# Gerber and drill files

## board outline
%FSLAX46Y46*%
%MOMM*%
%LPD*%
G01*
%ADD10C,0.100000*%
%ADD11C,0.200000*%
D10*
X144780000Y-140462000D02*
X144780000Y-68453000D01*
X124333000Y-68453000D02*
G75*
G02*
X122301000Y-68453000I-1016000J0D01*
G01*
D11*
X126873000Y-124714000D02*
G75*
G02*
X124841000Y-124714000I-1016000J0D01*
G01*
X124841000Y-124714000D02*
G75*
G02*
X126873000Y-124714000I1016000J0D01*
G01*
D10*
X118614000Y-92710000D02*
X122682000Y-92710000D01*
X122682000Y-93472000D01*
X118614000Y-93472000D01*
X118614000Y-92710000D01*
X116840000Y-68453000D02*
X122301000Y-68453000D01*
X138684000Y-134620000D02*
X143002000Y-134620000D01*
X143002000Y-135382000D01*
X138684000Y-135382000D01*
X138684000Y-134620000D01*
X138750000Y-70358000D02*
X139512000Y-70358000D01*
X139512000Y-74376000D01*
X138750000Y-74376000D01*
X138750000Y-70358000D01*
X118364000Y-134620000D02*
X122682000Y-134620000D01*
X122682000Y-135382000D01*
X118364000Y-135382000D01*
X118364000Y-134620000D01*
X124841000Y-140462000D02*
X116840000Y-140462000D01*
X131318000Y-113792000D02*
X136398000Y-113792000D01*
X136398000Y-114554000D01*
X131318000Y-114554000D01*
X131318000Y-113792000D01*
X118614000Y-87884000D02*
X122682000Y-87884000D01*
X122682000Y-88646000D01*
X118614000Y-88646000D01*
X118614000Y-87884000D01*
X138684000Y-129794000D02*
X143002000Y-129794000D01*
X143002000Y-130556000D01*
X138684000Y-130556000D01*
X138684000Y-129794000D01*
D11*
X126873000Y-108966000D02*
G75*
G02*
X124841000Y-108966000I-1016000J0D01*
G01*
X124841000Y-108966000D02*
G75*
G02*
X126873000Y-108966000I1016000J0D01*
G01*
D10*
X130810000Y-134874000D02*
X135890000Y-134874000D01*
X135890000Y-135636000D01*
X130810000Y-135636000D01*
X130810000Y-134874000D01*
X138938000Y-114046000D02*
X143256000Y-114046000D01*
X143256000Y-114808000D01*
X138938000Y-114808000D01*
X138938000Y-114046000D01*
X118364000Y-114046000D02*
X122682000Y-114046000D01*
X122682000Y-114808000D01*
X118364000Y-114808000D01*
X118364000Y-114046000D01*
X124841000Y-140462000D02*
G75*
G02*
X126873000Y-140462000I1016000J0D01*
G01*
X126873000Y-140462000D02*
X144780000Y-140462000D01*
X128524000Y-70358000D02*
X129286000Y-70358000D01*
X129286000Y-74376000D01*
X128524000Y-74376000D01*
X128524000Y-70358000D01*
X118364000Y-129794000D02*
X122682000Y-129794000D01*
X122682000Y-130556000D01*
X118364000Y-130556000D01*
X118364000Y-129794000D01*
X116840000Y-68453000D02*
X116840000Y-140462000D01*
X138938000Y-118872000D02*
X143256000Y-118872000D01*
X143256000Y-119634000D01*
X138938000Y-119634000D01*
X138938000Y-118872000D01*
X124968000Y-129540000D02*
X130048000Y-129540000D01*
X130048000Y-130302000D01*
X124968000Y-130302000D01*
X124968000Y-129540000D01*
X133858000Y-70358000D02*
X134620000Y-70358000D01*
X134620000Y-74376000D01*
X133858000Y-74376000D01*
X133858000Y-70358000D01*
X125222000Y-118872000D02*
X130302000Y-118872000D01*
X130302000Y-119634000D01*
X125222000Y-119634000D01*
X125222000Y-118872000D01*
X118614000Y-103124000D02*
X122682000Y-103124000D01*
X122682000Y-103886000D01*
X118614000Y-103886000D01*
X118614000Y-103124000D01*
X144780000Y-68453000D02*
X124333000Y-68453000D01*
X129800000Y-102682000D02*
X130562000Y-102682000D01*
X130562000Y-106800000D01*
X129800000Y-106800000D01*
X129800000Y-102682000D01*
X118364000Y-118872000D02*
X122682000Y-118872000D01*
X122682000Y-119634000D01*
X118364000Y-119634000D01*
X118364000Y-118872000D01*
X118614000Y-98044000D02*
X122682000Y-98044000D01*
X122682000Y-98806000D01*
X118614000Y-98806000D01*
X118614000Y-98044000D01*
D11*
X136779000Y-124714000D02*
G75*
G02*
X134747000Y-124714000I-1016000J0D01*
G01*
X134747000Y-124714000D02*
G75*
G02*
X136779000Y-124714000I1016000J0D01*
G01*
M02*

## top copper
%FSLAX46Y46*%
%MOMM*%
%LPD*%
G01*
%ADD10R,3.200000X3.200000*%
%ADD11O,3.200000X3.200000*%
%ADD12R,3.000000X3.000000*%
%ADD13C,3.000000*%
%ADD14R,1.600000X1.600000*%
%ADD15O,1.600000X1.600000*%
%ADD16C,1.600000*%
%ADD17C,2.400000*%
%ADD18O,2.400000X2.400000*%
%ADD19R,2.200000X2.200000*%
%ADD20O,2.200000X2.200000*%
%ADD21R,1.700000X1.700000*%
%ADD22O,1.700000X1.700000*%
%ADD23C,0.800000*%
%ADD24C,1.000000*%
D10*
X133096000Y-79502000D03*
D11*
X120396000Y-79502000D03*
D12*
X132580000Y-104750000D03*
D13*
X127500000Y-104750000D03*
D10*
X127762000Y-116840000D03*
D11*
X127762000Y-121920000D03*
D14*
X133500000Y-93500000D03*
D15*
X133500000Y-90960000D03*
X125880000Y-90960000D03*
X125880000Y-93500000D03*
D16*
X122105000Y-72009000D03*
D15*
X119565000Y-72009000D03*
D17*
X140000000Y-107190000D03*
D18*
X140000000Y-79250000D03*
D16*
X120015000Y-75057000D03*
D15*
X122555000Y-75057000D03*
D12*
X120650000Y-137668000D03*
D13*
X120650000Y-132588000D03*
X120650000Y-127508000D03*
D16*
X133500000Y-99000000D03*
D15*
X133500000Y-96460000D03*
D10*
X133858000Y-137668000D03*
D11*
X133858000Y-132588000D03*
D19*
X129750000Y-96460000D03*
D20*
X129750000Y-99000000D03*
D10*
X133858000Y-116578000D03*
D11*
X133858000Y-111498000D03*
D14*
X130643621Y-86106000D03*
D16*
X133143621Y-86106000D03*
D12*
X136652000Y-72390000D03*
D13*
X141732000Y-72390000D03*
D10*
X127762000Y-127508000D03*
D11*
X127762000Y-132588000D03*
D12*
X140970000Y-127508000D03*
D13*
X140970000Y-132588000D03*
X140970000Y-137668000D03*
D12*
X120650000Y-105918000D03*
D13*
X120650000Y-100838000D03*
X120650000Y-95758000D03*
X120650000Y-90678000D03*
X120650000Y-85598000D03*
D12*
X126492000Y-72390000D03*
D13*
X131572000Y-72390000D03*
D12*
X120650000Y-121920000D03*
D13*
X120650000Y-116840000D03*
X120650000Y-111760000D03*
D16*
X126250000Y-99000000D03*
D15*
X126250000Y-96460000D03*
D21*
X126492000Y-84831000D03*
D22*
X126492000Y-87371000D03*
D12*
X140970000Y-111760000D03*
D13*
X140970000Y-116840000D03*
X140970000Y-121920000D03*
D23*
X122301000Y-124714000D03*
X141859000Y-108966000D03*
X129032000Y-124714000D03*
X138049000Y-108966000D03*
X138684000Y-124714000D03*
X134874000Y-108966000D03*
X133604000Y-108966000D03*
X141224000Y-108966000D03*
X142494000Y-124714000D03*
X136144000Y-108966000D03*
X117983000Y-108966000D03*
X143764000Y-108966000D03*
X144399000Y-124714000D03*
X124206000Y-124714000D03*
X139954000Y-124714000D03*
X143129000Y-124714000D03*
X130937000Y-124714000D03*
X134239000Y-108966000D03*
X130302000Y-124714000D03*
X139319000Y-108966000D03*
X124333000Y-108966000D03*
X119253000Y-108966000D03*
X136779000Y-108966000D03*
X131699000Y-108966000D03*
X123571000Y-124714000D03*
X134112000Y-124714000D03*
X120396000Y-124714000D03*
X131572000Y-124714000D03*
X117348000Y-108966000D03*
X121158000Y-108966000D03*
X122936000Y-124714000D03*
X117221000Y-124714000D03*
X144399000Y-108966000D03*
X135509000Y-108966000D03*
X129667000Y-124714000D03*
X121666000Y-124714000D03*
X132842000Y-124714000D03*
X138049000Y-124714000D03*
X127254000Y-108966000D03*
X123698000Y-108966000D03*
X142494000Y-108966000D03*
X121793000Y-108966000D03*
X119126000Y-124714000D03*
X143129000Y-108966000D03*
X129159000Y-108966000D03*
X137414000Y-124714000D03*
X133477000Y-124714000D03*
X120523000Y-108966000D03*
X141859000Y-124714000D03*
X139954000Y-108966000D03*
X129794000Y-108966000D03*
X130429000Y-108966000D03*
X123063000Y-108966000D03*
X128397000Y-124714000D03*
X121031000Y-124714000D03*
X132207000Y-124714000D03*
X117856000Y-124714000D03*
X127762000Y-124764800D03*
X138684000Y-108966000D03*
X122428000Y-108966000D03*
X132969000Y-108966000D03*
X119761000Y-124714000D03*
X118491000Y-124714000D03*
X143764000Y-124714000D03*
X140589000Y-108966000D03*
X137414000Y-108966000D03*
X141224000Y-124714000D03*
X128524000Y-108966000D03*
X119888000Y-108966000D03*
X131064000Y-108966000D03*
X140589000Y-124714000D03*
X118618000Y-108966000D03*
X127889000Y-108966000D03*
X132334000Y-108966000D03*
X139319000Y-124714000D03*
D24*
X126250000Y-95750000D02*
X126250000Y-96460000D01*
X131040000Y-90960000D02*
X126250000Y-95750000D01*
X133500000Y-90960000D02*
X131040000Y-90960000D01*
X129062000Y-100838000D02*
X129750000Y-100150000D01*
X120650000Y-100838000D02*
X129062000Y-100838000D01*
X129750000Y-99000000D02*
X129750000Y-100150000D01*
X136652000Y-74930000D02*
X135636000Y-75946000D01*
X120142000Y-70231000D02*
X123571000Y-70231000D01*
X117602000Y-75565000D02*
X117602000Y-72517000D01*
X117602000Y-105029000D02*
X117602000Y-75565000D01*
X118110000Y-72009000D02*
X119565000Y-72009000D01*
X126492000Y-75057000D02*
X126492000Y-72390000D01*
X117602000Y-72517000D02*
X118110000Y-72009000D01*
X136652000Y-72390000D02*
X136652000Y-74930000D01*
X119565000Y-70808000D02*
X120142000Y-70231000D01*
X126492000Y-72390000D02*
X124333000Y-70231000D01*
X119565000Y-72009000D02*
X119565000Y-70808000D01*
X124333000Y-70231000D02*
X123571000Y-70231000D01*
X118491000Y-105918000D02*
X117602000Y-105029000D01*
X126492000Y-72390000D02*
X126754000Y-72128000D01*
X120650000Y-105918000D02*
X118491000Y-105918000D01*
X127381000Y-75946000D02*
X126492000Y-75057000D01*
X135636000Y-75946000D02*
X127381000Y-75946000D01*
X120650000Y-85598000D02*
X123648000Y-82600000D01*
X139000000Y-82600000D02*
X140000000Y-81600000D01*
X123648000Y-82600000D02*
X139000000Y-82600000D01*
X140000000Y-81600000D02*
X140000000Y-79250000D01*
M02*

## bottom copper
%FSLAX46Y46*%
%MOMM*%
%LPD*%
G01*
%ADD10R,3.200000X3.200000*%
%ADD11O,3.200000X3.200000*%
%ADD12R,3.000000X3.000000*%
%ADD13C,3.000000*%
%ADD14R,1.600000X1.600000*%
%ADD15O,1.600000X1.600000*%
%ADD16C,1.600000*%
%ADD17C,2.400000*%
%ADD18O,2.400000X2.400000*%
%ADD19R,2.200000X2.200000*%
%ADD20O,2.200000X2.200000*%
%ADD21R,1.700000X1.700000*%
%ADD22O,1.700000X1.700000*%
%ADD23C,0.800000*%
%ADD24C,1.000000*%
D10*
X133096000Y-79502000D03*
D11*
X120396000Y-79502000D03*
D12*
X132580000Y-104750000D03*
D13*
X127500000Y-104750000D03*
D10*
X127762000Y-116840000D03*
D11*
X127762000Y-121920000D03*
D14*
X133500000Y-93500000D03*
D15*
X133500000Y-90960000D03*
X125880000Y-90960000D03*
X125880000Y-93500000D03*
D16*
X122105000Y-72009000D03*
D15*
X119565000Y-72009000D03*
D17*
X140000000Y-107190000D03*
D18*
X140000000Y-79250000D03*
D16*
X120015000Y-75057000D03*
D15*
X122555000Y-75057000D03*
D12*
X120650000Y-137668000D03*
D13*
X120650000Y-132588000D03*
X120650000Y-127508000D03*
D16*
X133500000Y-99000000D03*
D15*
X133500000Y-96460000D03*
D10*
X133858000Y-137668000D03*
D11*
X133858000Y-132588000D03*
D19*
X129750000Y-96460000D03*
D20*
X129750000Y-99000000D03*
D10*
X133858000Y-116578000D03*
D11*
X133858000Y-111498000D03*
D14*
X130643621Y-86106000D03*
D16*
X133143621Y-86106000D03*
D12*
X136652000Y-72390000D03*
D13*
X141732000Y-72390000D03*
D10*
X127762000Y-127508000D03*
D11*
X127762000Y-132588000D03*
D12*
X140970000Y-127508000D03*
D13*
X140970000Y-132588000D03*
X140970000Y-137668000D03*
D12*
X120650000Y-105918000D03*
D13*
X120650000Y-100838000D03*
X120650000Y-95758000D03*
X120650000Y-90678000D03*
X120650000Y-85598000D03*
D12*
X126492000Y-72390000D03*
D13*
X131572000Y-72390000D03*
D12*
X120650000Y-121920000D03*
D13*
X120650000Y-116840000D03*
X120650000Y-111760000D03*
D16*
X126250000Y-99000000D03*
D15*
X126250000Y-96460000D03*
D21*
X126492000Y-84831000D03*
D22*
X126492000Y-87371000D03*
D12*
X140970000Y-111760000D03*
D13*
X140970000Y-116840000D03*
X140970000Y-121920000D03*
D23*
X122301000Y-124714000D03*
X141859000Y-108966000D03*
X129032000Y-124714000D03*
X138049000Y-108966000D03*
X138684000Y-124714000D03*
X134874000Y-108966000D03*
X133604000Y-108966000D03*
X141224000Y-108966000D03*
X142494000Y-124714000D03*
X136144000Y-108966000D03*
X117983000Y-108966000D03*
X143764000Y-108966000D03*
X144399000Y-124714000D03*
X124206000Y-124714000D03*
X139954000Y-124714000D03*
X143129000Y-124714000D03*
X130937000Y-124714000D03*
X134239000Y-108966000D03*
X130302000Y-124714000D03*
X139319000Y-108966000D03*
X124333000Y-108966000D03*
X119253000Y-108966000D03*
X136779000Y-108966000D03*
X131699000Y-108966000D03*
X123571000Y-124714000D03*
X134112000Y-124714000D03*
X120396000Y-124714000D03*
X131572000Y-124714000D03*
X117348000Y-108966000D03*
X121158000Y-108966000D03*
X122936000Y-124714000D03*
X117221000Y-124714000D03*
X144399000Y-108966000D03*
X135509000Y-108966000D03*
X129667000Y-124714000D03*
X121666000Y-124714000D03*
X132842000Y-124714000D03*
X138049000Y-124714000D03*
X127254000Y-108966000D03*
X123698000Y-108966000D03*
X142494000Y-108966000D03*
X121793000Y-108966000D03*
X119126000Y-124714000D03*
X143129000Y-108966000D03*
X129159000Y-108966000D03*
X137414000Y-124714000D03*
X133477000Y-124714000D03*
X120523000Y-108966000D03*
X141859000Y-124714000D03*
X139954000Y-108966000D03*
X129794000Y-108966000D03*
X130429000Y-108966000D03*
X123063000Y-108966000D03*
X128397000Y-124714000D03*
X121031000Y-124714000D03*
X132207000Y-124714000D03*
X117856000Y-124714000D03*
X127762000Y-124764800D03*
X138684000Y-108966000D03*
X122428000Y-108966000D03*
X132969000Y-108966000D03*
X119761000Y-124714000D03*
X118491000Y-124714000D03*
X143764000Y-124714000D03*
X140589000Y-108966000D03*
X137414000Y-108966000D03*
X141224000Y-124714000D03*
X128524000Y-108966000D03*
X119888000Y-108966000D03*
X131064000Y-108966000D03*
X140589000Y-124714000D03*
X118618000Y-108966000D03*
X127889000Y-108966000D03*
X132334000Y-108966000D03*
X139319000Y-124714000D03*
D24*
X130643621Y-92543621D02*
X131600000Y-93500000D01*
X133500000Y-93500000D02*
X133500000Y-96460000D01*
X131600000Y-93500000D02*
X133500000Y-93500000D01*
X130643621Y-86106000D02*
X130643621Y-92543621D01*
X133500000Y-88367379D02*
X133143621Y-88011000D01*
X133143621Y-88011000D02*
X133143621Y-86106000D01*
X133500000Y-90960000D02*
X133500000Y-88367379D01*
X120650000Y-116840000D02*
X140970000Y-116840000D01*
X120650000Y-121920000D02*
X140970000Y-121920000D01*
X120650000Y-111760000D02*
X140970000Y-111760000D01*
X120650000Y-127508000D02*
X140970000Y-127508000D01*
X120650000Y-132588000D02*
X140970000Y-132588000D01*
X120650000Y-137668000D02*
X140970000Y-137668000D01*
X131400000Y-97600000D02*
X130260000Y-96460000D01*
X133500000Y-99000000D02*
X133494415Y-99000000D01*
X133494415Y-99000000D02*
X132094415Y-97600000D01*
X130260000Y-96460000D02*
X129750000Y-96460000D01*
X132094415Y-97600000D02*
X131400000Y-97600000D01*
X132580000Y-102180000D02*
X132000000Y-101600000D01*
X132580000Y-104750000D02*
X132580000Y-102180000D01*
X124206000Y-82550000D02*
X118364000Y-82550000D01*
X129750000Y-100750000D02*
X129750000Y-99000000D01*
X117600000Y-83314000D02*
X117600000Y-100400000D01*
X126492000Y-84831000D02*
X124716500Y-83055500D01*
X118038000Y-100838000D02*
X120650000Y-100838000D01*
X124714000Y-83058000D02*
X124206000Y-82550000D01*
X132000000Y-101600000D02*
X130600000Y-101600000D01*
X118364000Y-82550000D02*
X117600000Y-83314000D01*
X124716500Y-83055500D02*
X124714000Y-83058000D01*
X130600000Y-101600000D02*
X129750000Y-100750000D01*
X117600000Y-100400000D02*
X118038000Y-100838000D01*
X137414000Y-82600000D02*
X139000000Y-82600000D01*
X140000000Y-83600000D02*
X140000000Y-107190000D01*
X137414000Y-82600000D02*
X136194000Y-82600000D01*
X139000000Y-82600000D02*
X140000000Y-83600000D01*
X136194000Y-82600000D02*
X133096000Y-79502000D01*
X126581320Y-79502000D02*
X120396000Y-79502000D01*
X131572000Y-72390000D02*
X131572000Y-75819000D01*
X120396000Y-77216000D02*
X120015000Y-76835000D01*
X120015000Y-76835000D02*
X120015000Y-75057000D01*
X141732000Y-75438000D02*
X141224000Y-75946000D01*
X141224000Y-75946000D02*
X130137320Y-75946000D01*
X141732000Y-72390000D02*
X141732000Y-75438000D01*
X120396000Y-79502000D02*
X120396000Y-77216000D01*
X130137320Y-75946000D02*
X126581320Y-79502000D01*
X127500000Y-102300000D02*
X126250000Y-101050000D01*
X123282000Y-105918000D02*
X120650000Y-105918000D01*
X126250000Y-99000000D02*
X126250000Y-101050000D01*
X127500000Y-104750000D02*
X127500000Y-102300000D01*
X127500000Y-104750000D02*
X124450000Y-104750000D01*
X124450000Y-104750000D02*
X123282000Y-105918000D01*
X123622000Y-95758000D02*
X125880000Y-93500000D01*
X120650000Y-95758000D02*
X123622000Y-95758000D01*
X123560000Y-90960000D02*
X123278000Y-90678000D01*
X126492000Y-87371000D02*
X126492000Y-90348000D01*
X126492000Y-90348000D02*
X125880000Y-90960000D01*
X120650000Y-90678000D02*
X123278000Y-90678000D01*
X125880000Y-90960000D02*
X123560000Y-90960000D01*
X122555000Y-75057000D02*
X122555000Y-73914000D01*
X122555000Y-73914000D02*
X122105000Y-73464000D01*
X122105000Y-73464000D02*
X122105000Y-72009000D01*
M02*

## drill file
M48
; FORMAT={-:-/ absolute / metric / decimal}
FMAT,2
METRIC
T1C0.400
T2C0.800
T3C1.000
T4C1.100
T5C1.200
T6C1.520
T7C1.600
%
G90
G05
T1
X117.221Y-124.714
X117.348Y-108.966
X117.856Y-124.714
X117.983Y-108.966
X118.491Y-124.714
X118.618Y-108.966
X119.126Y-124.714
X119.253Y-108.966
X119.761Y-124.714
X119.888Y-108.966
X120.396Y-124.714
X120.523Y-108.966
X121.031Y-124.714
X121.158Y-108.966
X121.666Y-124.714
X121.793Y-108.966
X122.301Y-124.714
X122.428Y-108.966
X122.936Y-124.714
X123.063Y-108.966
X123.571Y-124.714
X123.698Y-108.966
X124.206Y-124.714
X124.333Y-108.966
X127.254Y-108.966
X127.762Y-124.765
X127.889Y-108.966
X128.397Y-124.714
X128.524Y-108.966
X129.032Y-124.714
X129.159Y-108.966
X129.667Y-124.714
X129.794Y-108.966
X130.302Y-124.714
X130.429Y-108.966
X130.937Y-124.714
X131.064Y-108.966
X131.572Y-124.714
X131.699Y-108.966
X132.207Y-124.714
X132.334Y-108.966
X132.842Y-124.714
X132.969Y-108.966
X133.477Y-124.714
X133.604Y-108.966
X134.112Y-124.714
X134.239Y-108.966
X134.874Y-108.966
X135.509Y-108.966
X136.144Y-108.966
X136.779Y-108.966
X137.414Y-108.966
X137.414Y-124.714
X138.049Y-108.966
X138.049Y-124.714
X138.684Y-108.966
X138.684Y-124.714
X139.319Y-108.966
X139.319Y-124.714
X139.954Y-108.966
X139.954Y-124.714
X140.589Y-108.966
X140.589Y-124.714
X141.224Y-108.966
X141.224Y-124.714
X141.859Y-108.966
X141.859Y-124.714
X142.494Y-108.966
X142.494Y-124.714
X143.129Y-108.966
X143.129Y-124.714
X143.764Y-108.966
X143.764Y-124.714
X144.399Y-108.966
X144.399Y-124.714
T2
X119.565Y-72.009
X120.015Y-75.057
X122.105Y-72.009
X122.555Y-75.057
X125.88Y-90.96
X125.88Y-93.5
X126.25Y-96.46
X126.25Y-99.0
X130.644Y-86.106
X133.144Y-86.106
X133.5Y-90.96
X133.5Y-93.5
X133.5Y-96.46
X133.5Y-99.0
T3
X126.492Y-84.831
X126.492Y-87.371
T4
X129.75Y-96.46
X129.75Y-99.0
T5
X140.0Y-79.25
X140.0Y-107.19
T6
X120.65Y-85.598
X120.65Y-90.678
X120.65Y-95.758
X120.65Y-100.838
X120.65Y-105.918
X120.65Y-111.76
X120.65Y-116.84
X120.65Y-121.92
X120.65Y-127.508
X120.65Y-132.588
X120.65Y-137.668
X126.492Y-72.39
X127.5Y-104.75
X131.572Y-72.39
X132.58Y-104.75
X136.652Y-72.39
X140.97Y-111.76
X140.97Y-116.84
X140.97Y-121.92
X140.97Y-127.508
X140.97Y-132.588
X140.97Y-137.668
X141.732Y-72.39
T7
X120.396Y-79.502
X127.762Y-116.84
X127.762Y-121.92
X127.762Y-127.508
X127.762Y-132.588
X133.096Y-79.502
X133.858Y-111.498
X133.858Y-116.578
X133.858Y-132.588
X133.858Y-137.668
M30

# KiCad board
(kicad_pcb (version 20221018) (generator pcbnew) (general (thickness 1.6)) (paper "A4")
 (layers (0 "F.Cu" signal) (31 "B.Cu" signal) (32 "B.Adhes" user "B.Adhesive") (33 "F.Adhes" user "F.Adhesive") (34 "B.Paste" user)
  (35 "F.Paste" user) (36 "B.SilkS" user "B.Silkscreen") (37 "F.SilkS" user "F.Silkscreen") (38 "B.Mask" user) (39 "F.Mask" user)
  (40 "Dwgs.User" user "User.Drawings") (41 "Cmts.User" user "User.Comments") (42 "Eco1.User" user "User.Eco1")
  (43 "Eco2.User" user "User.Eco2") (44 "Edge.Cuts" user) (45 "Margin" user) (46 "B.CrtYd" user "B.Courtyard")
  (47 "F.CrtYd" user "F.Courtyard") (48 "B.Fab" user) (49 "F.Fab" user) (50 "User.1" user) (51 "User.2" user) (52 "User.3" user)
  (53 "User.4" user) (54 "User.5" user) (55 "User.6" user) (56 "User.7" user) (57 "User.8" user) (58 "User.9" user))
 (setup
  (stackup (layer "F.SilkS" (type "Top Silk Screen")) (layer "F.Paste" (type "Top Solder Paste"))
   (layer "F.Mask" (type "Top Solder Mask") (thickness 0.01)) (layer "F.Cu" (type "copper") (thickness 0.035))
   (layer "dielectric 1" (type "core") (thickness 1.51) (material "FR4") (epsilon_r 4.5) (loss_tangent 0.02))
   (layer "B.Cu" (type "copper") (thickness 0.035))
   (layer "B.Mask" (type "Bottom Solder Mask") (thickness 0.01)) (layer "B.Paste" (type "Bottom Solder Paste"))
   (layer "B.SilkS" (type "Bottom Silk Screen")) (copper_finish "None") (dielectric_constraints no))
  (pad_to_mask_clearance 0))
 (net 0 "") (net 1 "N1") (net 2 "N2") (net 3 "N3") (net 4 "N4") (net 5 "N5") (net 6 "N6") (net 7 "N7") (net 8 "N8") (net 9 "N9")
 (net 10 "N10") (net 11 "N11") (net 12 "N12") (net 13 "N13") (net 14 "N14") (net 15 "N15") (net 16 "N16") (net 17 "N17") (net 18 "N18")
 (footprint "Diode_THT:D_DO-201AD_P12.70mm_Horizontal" (layer "F.Cu") (at 133.096 79.502 180)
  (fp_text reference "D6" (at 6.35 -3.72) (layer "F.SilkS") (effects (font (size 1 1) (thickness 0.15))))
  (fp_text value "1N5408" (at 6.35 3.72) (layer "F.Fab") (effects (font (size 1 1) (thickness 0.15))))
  (pad "1" thru_hole rect (at 0 0 180) (size 3.2 3.2) (drill 1.6) (layers "*.Cu" "*.Mask") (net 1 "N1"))
  (pad "2" thru_hole oval (at 12.7 0 180) (size 3.2 3.2) (drill 1.6) (layers "*.Cu" "*.Mask") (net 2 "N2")))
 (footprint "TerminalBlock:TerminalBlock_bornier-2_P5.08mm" (layer "F.Cu") (at 132.58 104.75 180)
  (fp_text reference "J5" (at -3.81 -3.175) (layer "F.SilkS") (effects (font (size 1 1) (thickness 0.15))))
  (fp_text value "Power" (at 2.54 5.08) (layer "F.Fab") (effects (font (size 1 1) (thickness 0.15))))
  (pad "1" thru_hole rect (at 0 0 180) (size 3 3) (drill 1.52) (layers "*.Cu" "*.Mask") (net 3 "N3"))
  (pad "2" thru_hole circle (at 5.08 0 180) (size 3 3) (drill 1.52) (layers "*.Cu" "*.Mask") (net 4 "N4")))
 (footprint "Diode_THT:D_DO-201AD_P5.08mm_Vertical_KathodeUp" (layer "F.Cu") (at 127.762 116.84 -90)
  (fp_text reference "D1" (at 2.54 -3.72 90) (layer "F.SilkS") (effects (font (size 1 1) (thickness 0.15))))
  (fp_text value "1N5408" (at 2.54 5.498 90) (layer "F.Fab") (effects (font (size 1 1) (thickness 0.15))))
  (pad "1" thru_hole rect (at 0 0 270) (size 3.2 3.2) (drill 1.6) (layers "*.Cu" "*.Mask") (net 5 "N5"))
  (pad "2" thru_hole oval (at 5.08 0 270) (size 3.2 3.2) (drill 1.6) (layers "*.Cu" "*.Mask") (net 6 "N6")))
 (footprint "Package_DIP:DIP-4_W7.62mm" (layer "F.Cu") (at 133.5 93.5 180)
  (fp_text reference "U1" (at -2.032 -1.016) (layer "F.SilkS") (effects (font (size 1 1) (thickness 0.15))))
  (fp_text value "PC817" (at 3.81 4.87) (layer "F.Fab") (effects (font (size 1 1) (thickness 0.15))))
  (pad "1" thru_hole rect (at 0 0 180) (size 1.6 1.6) (drill 0.8) (layers "*.Cu" "*.Mask") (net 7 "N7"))
  (pad "2" thru_hole oval (at 0 2.54 180) (size 1.6 1.6) (drill 0.8) (layers "*.Cu" "*.Mask") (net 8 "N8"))
  (pad "3" thru_hole oval (at 7.62 2.54 180) (size 1.6 1.6) (drill 0.8) (layers "*.Cu" "*.Mask") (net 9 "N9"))
  (pad "4" thru_hole oval (at 7.62 0 180) (size 1.6 1.6) (drill 0.8) (layers "*.Cu" "*.Mask") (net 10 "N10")))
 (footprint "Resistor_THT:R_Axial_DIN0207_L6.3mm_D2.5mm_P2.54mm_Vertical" (layer "F.Cu") (at 122.105 72.009 180)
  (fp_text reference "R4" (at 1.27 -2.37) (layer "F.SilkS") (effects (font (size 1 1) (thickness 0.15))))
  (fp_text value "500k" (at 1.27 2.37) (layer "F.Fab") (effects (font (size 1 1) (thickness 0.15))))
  (pad "1" thru_hole circle (at 0 0 180) (size 1.6 1.6) (drill 0.8) (layers "*.Cu" "*.Mask") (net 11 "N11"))
  (pad "2" thru_hole oval (at 2.54 0 180) (size 1.6 1.6) (drill 0.8) (layers "*.Cu" "*.Mask") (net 4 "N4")))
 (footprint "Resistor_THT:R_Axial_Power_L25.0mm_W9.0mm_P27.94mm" (layer "F.Cu") (at 140 107.19 90)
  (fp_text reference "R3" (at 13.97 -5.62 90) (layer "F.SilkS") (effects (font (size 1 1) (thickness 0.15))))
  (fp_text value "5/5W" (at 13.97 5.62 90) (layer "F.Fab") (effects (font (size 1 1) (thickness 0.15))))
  (pad "1" thru_hole circle (at 0 0 90) (size 2.4 2.4) (drill 1.2) (layers "*.Cu" "*.Mask") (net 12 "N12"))
  (pad "2" thru_hole oval (at 27.94 0 90) (size 2.4 2.4) (drill 1.2) (layers "*.Cu" "*.Mask") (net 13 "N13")))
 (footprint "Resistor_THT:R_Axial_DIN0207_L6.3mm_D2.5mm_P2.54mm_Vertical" (layer "F.Cu") (at 120.015 75.057)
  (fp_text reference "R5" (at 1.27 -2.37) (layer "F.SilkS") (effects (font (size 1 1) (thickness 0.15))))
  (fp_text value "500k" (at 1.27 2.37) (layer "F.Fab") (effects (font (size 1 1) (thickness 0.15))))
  (pad "1" thru_hole circle (at 0 0) (size 1.6 1.6) (drill 0.8) (layers "*.Cu" "*.Mask") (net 2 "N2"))
  (pad "2" thru_hole oval (at 2.54 0) (size 1.6 1.6) (drill 0.8) (layers "*.Cu" "*.Mask") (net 11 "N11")))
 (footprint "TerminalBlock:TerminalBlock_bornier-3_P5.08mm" (layer "F.Cu") (at 120.65 137.668 90)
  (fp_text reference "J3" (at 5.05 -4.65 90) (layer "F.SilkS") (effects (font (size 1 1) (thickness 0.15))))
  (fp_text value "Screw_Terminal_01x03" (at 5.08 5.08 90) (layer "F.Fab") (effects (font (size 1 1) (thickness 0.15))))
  (pad "1" thru_hole rect (at 0 0 90) (size 3 3) (drill 1.52) (layers "*.Cu" "*.Mask") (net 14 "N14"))
  (pad "2" thru_hole circle (at 5.08 0 90) (size 3 3) (drill 1.52) (layers "*.Cu" "*.Mask") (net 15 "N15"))
  (pad "3" thru_hole circle (at 10.16 0 90) (size 3 3) (drill 1.52) (layers "*.Cu" "*.Mask") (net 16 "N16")))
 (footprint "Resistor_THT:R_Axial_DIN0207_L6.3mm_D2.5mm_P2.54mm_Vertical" (layer "F.Cu") (at 133.5 99 90)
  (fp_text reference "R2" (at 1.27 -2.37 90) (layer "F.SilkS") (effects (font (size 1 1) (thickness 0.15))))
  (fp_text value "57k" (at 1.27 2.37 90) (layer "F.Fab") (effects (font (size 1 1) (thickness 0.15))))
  (pad "1" thru_hole circle (at 0 0 90) (size 1.6 1.6) (drill 0.8) (layers "*.Cu" "*.Mask") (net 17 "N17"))
  (pad "2" thru_hole oval (at 2.54 0 90) (size 1.6 1.6) (drill 0.8) (layers "*.Cu" "*.Mask") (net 7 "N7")))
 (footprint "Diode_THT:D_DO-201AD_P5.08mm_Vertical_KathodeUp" (layer "F.Cu") (at 133.858 137.668 90)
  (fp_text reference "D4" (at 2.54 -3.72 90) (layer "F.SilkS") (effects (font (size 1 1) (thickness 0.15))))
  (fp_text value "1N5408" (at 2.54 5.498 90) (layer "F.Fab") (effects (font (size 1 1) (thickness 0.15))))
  (pad "1" thru_hole rect (at 0 0 90) (size 3.2 3.2) (drill 1.6) (layers "*.Cu" "*.Mask") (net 14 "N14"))
  (pad "2" thru_hole oval (at 5.08 0 90) (size 3.2 3.2) (drill 1.6) (layers "*.Cu" "*.Mask") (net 15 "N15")))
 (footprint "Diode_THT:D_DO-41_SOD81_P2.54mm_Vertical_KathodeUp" (layer "F.Cu") (at 129.75 96.46 -90)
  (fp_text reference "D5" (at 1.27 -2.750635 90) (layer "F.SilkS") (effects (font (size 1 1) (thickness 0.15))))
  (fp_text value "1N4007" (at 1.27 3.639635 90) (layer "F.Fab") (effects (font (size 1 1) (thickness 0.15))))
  (pad "1" thru_hole rect (at 0 0 270) (size 2.2 2.2) (drill 1.1) (layers "*.Cu" "*.Mask") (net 17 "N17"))
  (pad "2" thru_hole oval (at 2.54 0 270) (size 2.2 2.2) (drill 1.1) (layers "*.Cu" "*.Mask") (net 3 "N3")))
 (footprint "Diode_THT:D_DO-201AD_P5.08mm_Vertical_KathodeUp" (layer "F.Cu") (at 133.858 116.578 90)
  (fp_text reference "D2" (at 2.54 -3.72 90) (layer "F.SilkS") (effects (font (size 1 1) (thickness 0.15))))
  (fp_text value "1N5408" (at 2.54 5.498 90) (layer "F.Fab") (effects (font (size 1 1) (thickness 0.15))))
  (pad "1" thru_hole rect (at 0 0 90) (size 3.2 3.2) (drill 1.6) (layers "*.Cu" "*.Mask") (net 5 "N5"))
  (pad "2" thru_hole oval (at 5.08 0 90) (size 3.2 3.2) (drill 1.6) (layers "*.Cu" "*.Mask") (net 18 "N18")))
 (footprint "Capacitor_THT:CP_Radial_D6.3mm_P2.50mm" (layer "F.Cu") (at 130.643621 86.106)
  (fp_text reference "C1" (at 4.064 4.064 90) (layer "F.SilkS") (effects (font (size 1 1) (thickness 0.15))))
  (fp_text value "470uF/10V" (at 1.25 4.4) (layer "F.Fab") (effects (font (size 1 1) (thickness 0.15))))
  (pad "1" thru_hole rect (at 0 0) (size 1.6 1.6) (drill 0.8) (layers "*.Cu" "*.Mask") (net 7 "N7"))
  (pad "2" thru_hole circle (at 2.5 0) (size 1.6 1.6) (drill 0.8) (layers "*.Cu" "*.Mask") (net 8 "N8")))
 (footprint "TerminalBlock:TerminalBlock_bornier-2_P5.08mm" (layer "F.Cu") (at 136.652 72.39)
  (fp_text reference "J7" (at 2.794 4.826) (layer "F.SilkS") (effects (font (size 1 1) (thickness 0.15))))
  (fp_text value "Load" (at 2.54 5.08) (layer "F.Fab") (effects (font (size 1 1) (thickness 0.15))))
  (pad "1" thru_hole rect (at 0 0) (size 3 3) (drill 1.52) (layers "*.Cu" "*.Mask") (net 4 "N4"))
  (pad "2" thru_hole circle (at 5.08 0) (size 3 3) (drill 1.52) (layers "*.Cu" "*.Mask") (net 2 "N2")))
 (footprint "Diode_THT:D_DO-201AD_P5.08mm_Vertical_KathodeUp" (layer "F.Cu") (at 127.762 127.508 -90)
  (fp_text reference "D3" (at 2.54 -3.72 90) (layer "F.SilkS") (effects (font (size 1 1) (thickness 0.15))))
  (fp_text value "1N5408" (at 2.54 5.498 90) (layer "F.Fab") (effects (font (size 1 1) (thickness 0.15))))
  (pad "1" thru_hole rect (at 0 0 270) (size 3.2 3.2) (drill 1.6) (layers "*.Cu" "*.Mask") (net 16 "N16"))
  (pad "2" thru_hole oval (at 5.08 0 270) (size 3.2 3.2) (drill 1.6) (layers "*.Cu" "*.Mask") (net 15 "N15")))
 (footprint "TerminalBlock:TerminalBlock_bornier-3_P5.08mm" (layer "F.Cu") (at 140.97 127.508 -90)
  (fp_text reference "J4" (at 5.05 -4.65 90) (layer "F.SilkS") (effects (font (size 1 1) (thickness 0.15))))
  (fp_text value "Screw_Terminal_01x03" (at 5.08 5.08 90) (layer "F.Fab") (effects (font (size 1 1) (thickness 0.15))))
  (pad "1" thru_hole rect (at 0 0 270) (size 3 3) (drill 1.52) (layers "*.Cu" "*.Mask") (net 16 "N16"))
  (pad "2" thru_hole circle (at 5.08 0 270) (size 3 3) (drill 1.52) (layers "*.Cu" "*.Mask") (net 15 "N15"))
  (pad "3" thru_hole circle (at 10.16 0 270) (size 3 3) (drill 1.52) (layers "*.Cu" "*.Mask") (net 14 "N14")))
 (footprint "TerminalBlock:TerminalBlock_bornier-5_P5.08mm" (layer "F.Cu") (at 120.65 105.918 90)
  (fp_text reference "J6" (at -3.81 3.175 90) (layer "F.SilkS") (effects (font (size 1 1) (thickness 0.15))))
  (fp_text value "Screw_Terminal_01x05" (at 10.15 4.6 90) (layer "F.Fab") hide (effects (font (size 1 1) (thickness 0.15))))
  (pad "1" thru_hole rect (at 0 0 90) (size 3 3) (drill 1.52) (layers "*.Cu" "*.Mask") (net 4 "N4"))
  (pad "2" thru_hole circle (at 5.08 0 90) (size 3 3) (drill 1.52) (layers "*.Cu" "*.Mask") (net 3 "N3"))
  (pad "3" thru_hole circle (at 10.16 0 90) (size 3 3) (drill 1.52) (layers "*.Cu" "*.Mask") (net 10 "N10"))
  (pad "4" thru_hole circle (at 15.24 0 90) (size 3 3) (drill 1.52) (layers "*.Cu" "*.Mask") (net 9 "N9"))
  (pad "5" thru_hole circle (at 20.32 0 90) (size 3 3) (drill 1.52) (layers "*.Cu" "*.Mask") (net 13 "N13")))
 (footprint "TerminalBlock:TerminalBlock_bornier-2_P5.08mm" (layer "F.Cu") (at 126.492 72.39)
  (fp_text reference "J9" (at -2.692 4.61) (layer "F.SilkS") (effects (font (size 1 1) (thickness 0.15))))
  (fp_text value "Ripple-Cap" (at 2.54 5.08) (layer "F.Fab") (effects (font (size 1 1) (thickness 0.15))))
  (pad "1" thru_hole rect (at 0 0) (size 3 3) (drill 1.52) (layers "*.Cu" "*.Mask") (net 4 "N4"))
  (pad "2" thru_hole circle (at 5.08 0) (size 3 3) (drill 1.52) (layers "*.Cu" "*.Mask") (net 2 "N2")))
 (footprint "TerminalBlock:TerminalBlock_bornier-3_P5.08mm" (layer "F.Cu") (at 120.65 121.92 90)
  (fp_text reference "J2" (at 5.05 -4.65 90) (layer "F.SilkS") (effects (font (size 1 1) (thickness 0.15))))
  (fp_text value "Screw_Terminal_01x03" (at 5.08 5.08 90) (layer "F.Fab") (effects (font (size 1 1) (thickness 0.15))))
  (pad "1" thru_hole rect (at 0 0 90) (size 3 3) (drill 1.52) (layers "*.Cu" "*.Mask") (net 6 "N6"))
  (pad "2" thru_hole circle (at 5.08 0 90) (size 3 3) (drill 1.52) (layers "*.Cu" "*.Mask") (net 5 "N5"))
  (pad "3" thru_hole circle (at 10.16 0 90) (size 3 3) (drill 1.52) (layers "*.Cu" "*.Mask") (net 18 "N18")))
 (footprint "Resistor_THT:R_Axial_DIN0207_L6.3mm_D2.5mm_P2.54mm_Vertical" (layer "F.Cu") (at 126.25 99 90)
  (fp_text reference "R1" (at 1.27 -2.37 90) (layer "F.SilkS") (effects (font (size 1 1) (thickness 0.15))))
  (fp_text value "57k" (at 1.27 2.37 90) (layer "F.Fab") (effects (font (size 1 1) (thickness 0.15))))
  (pad "1" thru_hole circle (at 0 0 90) (size 1.6 1.6) (drill 0.8) (layers "*.Cu" "*.Mask") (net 4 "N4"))
  (pad "2" thru_hole oval (at 2.54 0 90) (size 1.6 1.6) (drill 0.8) (layers "*.Cu" "*.Mask") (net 8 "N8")))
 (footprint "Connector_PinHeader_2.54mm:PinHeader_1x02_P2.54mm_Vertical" (layer "F.Cu") (at 126.492 84.831)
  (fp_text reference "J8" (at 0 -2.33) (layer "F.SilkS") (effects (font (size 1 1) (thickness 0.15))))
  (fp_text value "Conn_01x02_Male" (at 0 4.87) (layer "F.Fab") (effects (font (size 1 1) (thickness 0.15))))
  (pad "1" thru_hole rect (at 0 0) (size 1.7 1.7) (drill 1) (layers "*.Cu" "*.Mask") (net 3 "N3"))
  (pad "2" thru_hole oval (at 0 2.54) (size 1.7 1.7) (drill 1) (layers "*.Cu" "*.Mask") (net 9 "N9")))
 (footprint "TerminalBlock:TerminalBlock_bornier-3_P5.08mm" (layer "F.Cu") (at 140.97 111.76 -90)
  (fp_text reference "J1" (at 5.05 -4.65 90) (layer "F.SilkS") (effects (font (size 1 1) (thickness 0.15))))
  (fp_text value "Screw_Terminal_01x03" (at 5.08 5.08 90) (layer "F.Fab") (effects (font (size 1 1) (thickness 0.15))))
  (pad "1" thru_hole rect (at 0 0 270) (size 3 3) (drill 1.52) (layers "*.Cu" "*.Mask") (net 18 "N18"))
  (pad "2" thru_hole circle (at 5.08 0 270) (size 3 3) (drill 1.52) (layers "*.Cu" "*.Mask") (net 5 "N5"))
  (pad "3" thru_hole circle (at 10.16 0 270) (size 3 3) (drill 1.52) (layers "*.Cu" "*.Mask") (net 6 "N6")))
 (gr_line (start 144.78 140.462) (end 144.78 68.453) (stroke (width 0.1) (type solid)) (layer "Edge.Cuts"))
 (gr_arc (start 124.333 68.453) (mid 123.317 69.469) (end 122.301 68.453) (stroke (width 0.1) (type solid)) (layer "Edge.Cuts"))
 (gr_circle (center 125.857 124.714) (end 126.873 124.714) (stroke (width 0.2) (type solid)) (fill none) (layer "Edge.Cuts"))
 (gr_rect (start 118.614 92.71) (end 122.682 93.472) (stroke (width 0.1) (type solid)) (fill none) (layer "Edge.Cuts"))
 (gr_line (start 116.84 68.453) (end 122.301 68.453) (stroke (width 0.1) (type solid)) (layer "Edge.Cuts"))
 (gr_rect (start 138.684 134.62) (end 143.002 135.382) (stroke (width 0.1) (type solid)) (fill none) (layer "Edge.Cuts"))
 (gr_rect (start 138.75 70.358) (end 139.512 74.376) (stroke (width 0.1) (type solid)) (fill none) (layer "Edge.Cuts"))
 (gr_rect (start 118.364 134.62) (end 122.682 135.382) (stroke (width 0.1) (type solid)) (fill none) (layer "Edge.Cuts"))
 (gr_line (start 124.841 140.462) (end 116.84 140.462) (stroke (width 0.1) (type solid)) (layer "Edge.Cuts"))
 (gr_rect (start 131.318 113.792) (end 136.398 114.554) (stroke (width 0.1) (type solid)) (fill none) (layer "Edge.Cuts"))
 (gr_rect (start 118.614 87.884) (end 122.682 88.646) (stroke (width 0.1) (type solid)) (fill none) (layer "Edge.Cuts"))
 (gr_rect (start 138.684 129.794) (end 143.002 130.556) (stroke (width 0.1) (type solid)) (fill none) (layer "Edge.Cuts"))
 (gr_circle (center 125.857 108.966) (end 126.873 108.966) (stroke (width 0.2) (type solid)) (fill none) (layer "Edge.Cuts"))
 (gr_rect (start 130.81 134.874) (end 135.89 135.636) (stroke (width 0.1) (type solid)) (fill none) (layer "Edge.Cuts"))
 (gr_rect (start 138.938 114.046) (end 143.256 114.808) (stroke (width 0.1) (type solid)) (fill none) (layer "Edge.Cuts"))
 (gr_rect (start 118.364 114.046) (end 122.682 114.808) (stroke (width 0.1) (type solid)) (fill none) (layer "Edge.Cuts"))
 (gr_arc (start 124.841 140.462) (mid 125.857 139.446) (end 126.873 140.462) (stroke (width 0.1) (type solid)) (layer "Edge.Cuts"))
 (gr_line (start 126.873 140.462) (end 144.78 140.462) (stroke (width 0.1) (type solid)) (layer "Edge.Cuts"))
 (gr_rect (start 128.524 70.358) (end 129.286 74.376) (stroke (width 0.1) (type solid)) (fill none) (layer "Edge.Cuts"))
 (gr_rect (start 118.364 129.794) (end 122.682 130.556) (stroke (width 0.1) (type solid)) (fill none) (layer "Edge.Cuts"))
 (gr_line (start 116.84 68.453) (end 116.84 140.462) (stroke (width 0.1) (type solid)) (layer "Edge.Cuts"))
 (gr_rect (start 138.938 118.872) (end 143.256 119.634) (stroke (width 0.1) (type solid)) (fill none) (layer "Edge.Cuts"))
 (gr_rect (start 124.968 129.54) (end 130.048 130.302) (stroke (width 0.1) (type solid)) (fill none) (layer "Edge.Cuts"))
 (gr_rect (start 133.858 70.358) (end 134.62 74.376) (stroke (width 0.1) (type solid)) (fill none) (layer "Edge.Cuts"))
 (gr_rect (start 125.222 118.872) (end 130.302 119.634) (stroke (width 0.1) (type solid)) (fill none) (layer "Edge.Cuts"))
 (gr_rect (start 118.614 103.124) (end 122.682 103.886) (stroke (width 0.1) (type solid)) (fill none) (layer "Edge.Cuts"))
 (gr_line (start 144.78 68.453) (end 124.333 68.453) (stroke (width 0.1) (type solid)) (layer "Edge.Cuts"))
 (gr_rect (start 129.8 102.682) (end 130.562 106.8) (stroke (width 0.1) (type solid)) (fill none) (layer "Edge.Cuts"))
 (gr_rect (start 118.364 118.872) (end 122.682 119.634) (stroke (width 0.1) (type solid)) (fill none) (layer "Edge.Cuts"))
 (gr_rect (start 118.614 98.044) (end 122.682 98.806) (stroke (width 0.1) (type solid)) (fill none) (layer "Edge.Cuts"))
 (gr_circle (center 135.763 124.714) (end 136.779 124.714) (stroke (width 0.2) (type solid)) (fill none) (layer "Edge.Cuts"))
 (via (at 122.301 124.714) (size 0.8) (drill 0.4) (layers "F.Cu" "B.Cu") (free) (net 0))
 (via (at 141.859 108.966) (size 0.8) (drill 0.4) (layers "F.Cu" "B.Cu") (free) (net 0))
 (via (at 129.032 124.714) (size 0.8) (drill 0.4) (layers "F.Cu" "B.Cu") (free) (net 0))
 (via (at 138.049 108.966) (size 0.8) (drill 0.4) (layers "F.Cu" "B.Cu") (free) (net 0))
 (via (at 138.684 124.714) (size 0.8) (drill 0.4) (layers "F.Cu" "B.Cu") (free) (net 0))
 (via (at 134.874 108.966) (size 0.8) (drill 0.4) (layers "F.Cu" "B.Cu") (free) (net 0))
 (via (at 133.604 108.966) (size 0.8) (drill 0.4) (layers "F.Cu" "B.Cu") (free) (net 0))
 (via (at 141.224 108.966) (size 0.8) (drill 0.4) (layers "F.Cu" "B.Cu") (free) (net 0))
 (via (at 142.494 124.714) (size 0.8) (drill 0.4) (layers "F.Cu" "B.Cu") (free) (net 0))
 (via (at 136.144 108.966) (size 0.8) (drill 0.4) (layers "F.Cu" "B.Cu") (free) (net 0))
 (via (at 117.983 108.966) (size 0.8) (drill 0.4) (layers "F.Cu" "B.Cu") (free) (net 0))
 (via (at 143.764 108.966) (size 0.8) (drill 0.4) (layers "F.Cu" "B.Cu") (free) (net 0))
 (via (at 144.399 124.714) (size 0.8) (drill 0.4) (layers "F.Cu" "B.Cu") (free) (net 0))
 (via (at 124.206 124.714) (size 0.8) (drill 0.4) (layers "F.Cu" "B.Cu") (free) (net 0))
 (via (at 139.954 124.714) (size 0.8) (drill 0.4) (layers "F.Cu" "B.Cu") (free) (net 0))
 (via (at 143.129 124.714) (size 0.8) (drill 0.4) (layers "F.Cu" "B.Cu") (free) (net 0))
 (via (at 130.937 124.714) (size 0.8) (drill 0.4) (layers "F.Cu" "B.Cu") (free) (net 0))
 (via (at 134.239 108.966) (size 0.8) (drill 0.4) (layers "F.Cu" "B.Cu") (free) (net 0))
 (via (at 130.302 124.714) (size 0.8) (drill 0.4) (layers "F.Cu" "B.Cu") (free) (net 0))
 (via (at 139.319 108.966) (size 0.8) (drill 0.4) (layers "F.Cu" "B.Cu") (free) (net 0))
 (via (at 124.333 108.966) (size 0.8) (drill 0.4) (layers "F.Cu" "B.Cu") (free) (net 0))
 (via (at 119.253 108.966) (size 0.8) (drill 0.4) (layers "F.Cu" "B.Cu") (free) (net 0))
 (via (at 136.779 108.966) (size 0.8) (drill 0.4) (layers "F.Cu" "B.Cu") (free) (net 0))
 (via (at 131.699 108.966) (size 0.8) (drill 0.4) (layers "F.Cu" "B.Cu") (free) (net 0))
 (via (at 123.571 124.714) (size 0.8) (drill 0.4) (layers "F.Cu" "B.Cu") (free) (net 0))
 (via (at 134.112 124.714) (size 0.8) (drill 0.4) (layers "F.Cu" "B.Cu") (free) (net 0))
 (via (at 120.396 124.714) (size 0.8) (drill 0.4) (layers "F.Cu" "B.Cu") (free) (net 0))
 (via (at 131.572 124.714) (size 0.8) (drill 0.4) (layers "F.Cu" "B.Cu") (free) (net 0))
 (via (at 117.348 108.966) (size 0.8) (drill 0.4) (layers "F.Cu" "B.Cu") (remove_unused_layers) (keep_end_layers) (free)
  (zone_layer_connections) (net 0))
 (via (at 121.158 108.966) (size 0.8) (drill 0.4) (layers "F.Cu" "B.Cu") (free) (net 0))
 (via (at 122.936 124.714) (size 0.8) (drill 0.4) (layers "F.Cu" "B.Cu") (free) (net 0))
 (via (at 117.221 124.714) (size 0.8) (drill 0.4) (layers "F.Cu" "B.Cu") (free) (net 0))
 (via (at 144.399 108.966) (size 0.8) (drill 0.4) (layers "F.Cu" "B.Cu") (free) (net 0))
 (via (at 135.509 108.966) (size 0.8) (drill 0.4) (layers "F.Cu" "B.Cu") (free) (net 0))
 (via (at 129.667 124.714) (size 0.8) (drill 0.4) (layers "F.Cu" "B.Cu") (free) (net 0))
 (via (at 121.666 124.714) (size 0.8) (drill 0.4) (layers "F.Cu" "B.Cu") (free) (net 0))
 (via (at 132.842 124.714) (size 0.8) (drill 0.4) (layers "F.Cu" "B.Cu") (free) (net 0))
 (via (at 138.049 124.714) (size 0.8) (drill 0.4) (layers "F.Cu" "B.Cu") (free) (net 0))
 (via (at 127.254 108.966) (size 0.8) (drill 0.4) (layers "F.Cu" "B.Cu") (free) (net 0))
 (via (at 123.698 108.966) (size 0.8) (drill 0.4) (layers "F.Cu" "B.Cu") (free) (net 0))
 (via (at 142.494 108.966) (size 0.8) (drill 0.4) (layers "F.Cu" "B.Cu") (free) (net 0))
 (via (at 121.793 108.966) (size 0.8) (drill 0.4) (layers "F.Cu" "B.Cu") (free) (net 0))
 (via (at 119.126 124.714) (size 0.8) (drill 0.4) (layers "F.Cu" "B.Cu") (free) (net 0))
 (via (at 143.129 108.966) (size 0.8) (drill 0.4) (layers "F.Cu" "B.Cu") (free) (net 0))
 (via (at 129.159 108.966) (size 0.8) (drill 0.4) (layers "F.Cu" "B.Cu") (free) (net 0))
 (via (at 137.414 124.714) (size 0.8) (drill 0.4) (layers "F.Cu" "B.Cu") (free) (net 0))
 (via (at 133.477 124.714) (size 0.8) (drill 0.4) (layers "F.Cu" "B.Cu") (free) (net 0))
 (via (at 120.523 108.966) (size 0.8) (drill 0.4) (layers "F.Cu" "B.Cu") (free) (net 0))
 (via (at 141.859 124.714) (size 0.8) (drill 0.4) (layers "F.Cu" "B.Cu") (free) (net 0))
 (via (at 139.954 108.966) (size 0.8) (drill 0.4) (layers "F.Cu" "B.Cu") (free) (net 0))
 (via (at 129.794 108.966) (size 0.8) (drill 0.4) (layers "F.Cu" "B.Cu") (free) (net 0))
 (via (at 130.429 108.966) (size 0.8) (drill 0.4) (layers "F.Cu" "B.Cu") (free) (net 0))
 (via (at 123.063 108.966) (size 0.8) (drill 0.4) (layers "F.Cu" "B.Cu") (free) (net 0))
 (via (at 128.397 124.714) (size 0.8) (drill 0.4) (layers "F.Cu" "B.Cu") (free) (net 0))
 (via (at 121.031 124.714) (size 0.8) (drill 0.4) (layers "F.Cu" "B.Cu") (free) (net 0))
 (via (at 132.207 124.714) (size 0.8) (drill 0.4) (layers "F.Cu" "B.Cu") (free) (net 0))
 (via (at 117.856 124.714) (size 0.8) (drill 0.4) (layers "F.Cu" "B.Cu") (free) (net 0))
 (via (at 127.762 124.7648) (size 0.8) (drill 0.4) (layers "F.Cu" "B.Cu") (free) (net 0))
 (via (at 138.684 108.966) (size 0.8) (drill 0.4) (layers "F.Cu" "B.Cu") (free) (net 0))
 (via (at 122.428 108.966) (size 0.8) (drill 0.4) (layers "F.Cu" "B.Cu") (free) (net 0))
 (via (at 132.969 108.966) (size 0.8) (drill 0.4) (layers "F.Cu" "B.Cu") (free) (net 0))
 (via (at 119.761 124.714) (size 0.8) (drill 0.4) (layers "F.Cu" "B.Cu") (free) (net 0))
 (via (at 118.491 124.714) (size 0.8) (drill 0.4) (layers "F.Cu" "B.Cu") (free) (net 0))
 (via (at 143.764 124.714) (size 0.8) (drill 0.4) (layers "F.Cu" "B.Cu") (free) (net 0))
 (via (at 140.589 108.966) (size 0.8) (drill 0.4) (layers "F.Cu" "B.Cu") (free) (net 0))
 (via (at 137.414 108.966) (size 0.8) (drill 0.4) (layers "F.Cu" "B.Cu") (free) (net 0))
 (via (at 141.224 124.714) (size 0.8) (drill 0.4) (layers "F.Cu" "B.Cu") (free) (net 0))
 (via (at 128.524 108.966) (size 0.8) (drill 0.4) (layers "F.Cu" "B.Cu") (free) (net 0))
 (via (at 119.888 108.966) (size 0.8) (drill 0.4) (layers "F.Cu" "B.Cu") (free) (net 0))
 (via (at 131.064 108.966) (size 0.8) (drill 0.4) (layers "F.Cu" "B.Cu") (free) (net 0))
 (via (at 140.589 124.714) (size 0.8) (drill 0.4) (layers "F.Cu" "B.Cu") (free) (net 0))
 (via (at 118.618 108.966) (size 0.8) (drill 0.4) (layers "F.Cu" "B.Cu") (free) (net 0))
 (via (at 127.889 108.966) (size 0.8) (drill 0.4) (layers "F.Cu" "B.Cu") (free) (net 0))
 (via (at 132.334 108.966) (size 0.8) (drill 0.4) (layers "F.Cu" "B.Cu") (free) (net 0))
 (via (at 139.319 124.714) (size 0.8) (drill 0.4) (layers "F.Cu" "B.Cu") (free) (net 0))
 (segment (start 130.643621 92.543621) (end 131.6 93.5) (width 1) (layer "B.Cu") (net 7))
 (segment (start 133.5 93.5) (end 133.5 96.46) (width 1) (layer "B.Cu") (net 7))
 (segment (start 131.6 93.5) (end 133.5 93.5) (width 1) (layer "B.Cu") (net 7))
 (segment (start 130.643621 86.106) (end 130.643621 92.543621) (width 1) (layer "B.Cu") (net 7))
 (segment (start 126.25 95.75) (end 126.25 96.46) (width 1) (layer "F.Cu") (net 8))
 (segment (start 131.04 90.96) (end 126.25 95.75) (width 1) (layer "F.Cu") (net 8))
 (segment (start 133.5 90.96) (end 131.04 90.96) (width 1) (layer "F.Cu") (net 8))
 (segment (start 133.5 88.367379) (end 133.143621 88.011) (width 1) (layer "B.Cu") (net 8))
 (segment (start 133.143621 88.011) (end 133.143621 86.106) (width 1) (layer "B.Cu") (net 8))
 (segment (start 133.5 90.96) (end 133.5 88.367379) (width 1) (layer "B.Cu") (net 8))
 (segment (start 120.65 116.84) (end 140.97 116.84) (width 1) (layer "B.Cu") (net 5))
 (segment (start 120.65 121.92) (end 140.97 121.92) (width 1) (layer "B.Cu") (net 6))
 (segment (start 120.65 111.76) (end 140.97 111.76) (width 1) (layer "B.Cu") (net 18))
 (segment (start 120.65 127.508) (end 140.97 127.508) (width 1) (layer "B.Cu") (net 16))
 (segment (start 120.65 132.588) (end 140.97 132.588) (width 1) (layer "B.Cu") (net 15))
 (segment (start 120.65 137.668) (end 140.97 137.668) (width 1) (layer "B.Cu") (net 14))
 (segment (start 131.4 97.6) (end 130.26 96.46) (width 1) (layer "B.Cu") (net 17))
 (segment (start 133.5 99) (end 133.494415 99) (width 1) (layer "B.Cu") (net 17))
 (segment (start 133.494415 99) (end 132.094415 97.6) (width 1) (layer "B.Cu") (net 17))
 (segment (start 130.26 96.46) (end 129.75 96.46) (width 1) (layer "B.Cu") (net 17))
 (segment (start 132.094415 97.6) (end 131.4 97.6) (width 1) (layer "B.Cu") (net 17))
 (segment (start 129.062 100.838) (end 129.75 100.15) (width 1) (layer "F.Cu") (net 3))
 (segment (start 120.65 100.838) (end 129.062 100.838) (width 1) (layer "F.Cu") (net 3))
 (segment (start 129.75 99) (end 129.75 100.15) (width 1) (layer "F.Cu") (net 3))
 (segment (start 132.58 102.18) (end 132 101.6) (width 1) (layer "B.Cu") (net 3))
 (segment (start 132.58 104.75) (end 132.58 102.18) (width 1) (layer "B.Cu") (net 3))
 (segment (start 124.206 82.55) (end 118.364 82.55) (width 1) (layer "B.Cu") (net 3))
 (segment (start 129.75 100.75) (end 129.75 99) (width 1) (layer "B.Cu") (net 3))
 (segment (start 117.6 83.314) (end 117.6 100.4) (width 1) (layer "B.Cu") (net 3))
 (segment (start 126.492 84.831) (end 124.7165 83.0555) (width 1) (layer "B.Cu") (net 3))
 (segment (start 118.038 100.838) (end 120.65 100.838) (width 1) (layer "B.Cu") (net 3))
 (segment (start 124.714 83.058) (end 124.206 82.55) (width 1) (layer "B.Cu") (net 3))
 (segment (start 132 101.6) (end 130.6 101.6) (width 1) (layer "B.Cu") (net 3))
 (segment (start 118.364 82.55) (end 117.6 83.314) (width 1) (layer "B.Cu") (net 3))
 (segment (start 124.7165 83.0555) (end 124.714 83.058) (width 1) (layer "B.Cu") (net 3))
 (segment (start 130.6 101.6) (end 129.75 100.75) (width 1) (layer "B.Cu") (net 3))
 (segment (start 117.6 100.4) (end 118.038 100.838) (width 1) (layer "B.Cu") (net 3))
 (segment (start 137.414 82.6) (end 139 82.6) (width 1) (layer "B.Cu") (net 1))
 (segment (start 140 83.6) (end 140 107.19) (width 1) (layer "B.Cu") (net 1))
 (segment (start 137.414 82.6) (end 136.194 82.6) (width 1) (layer "B.Cu") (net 1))
 (segment (start 139 82.6) (end 140 83.6) (width 1) (layer "B.Cu") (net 1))
 (segment (start 136.194 82.6) (end 133.096 79.502) (width 1) (layer "B.Cu") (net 1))
 (segment (start 126.58132 79.502) (end 120.396 79.502) (width 1) (layer "B.Cu") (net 2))
 (segment (start 131.572 72.39) (end 131.572 75.819) (width 1) (layer "B.Cu") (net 2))
 (segment (start 120.396 77.216) (end 120.015 76.835) (width 1) (layer "B.Cu") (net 2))
 (segment (start 120.015 76.835) (end 120.015 75.057) (width 1) (layer "B.Cu") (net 2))
 (segment (start 141.732 75.438) (end 141.224 75.946) (width 1) (layer "B.Cu") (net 2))
 (segment (start 141.224 75.946) (end 130.13732 75.946) (width 1) (layer "B.Cu") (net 2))
 (segment (start 141.732 72.39) (end 141.732 75.438) (width 1) (layer "B.Cu") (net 2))
 (segment (start 120.396 79.502) (end 120.396 77.216) (width 1) (layer "B.Cu") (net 2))
 (segment (start 130.13732 75.946) (end 126.58132 79.502) (width 1) (layer "B.Cu") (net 2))
 (segment (start 136.652 74.93) (end 135.636 75.946) (width 1) (layer "F.Cu") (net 4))
 (segment (start 120.142 70.231) (end 123.571 70.231) (width 1) (layer "F.Cu") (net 4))
 (segment (start 117.602 75.565) (end 117.602 72.517) (width 1) (layer "F.Cu") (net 4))
 (segment (start 117.602 105.029) (end 117.602 75.565) (width 1) (layer "F.Cu") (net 4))
 (segment (start 118.11 72.009) (end 119.565 72.009) (width 1) (layer "F.Cu") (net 4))
 (segment (start 126.492 75.057) (end 126.492 72.39) (width 1) (layer "F.Cu") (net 4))
 (segment (start 117.602 72.517) (end 118.11 72.009) (width 1) (layer "F.Cu") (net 4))
 (segment (start 136.652 72.39) (end 136.652 74.93) (width 1) (layer "F.Cu") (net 4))
 (segment (start 119.565 70.808) (end 120.142 70.231) (width 1) (layer "F.Cu") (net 4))
 (segment (start 126.492 72.39) (end 124.333 70.231) (width 1) (layer "F.Cu") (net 4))
 (segment (start 119.565 72.009) (end 119.565 70.808) (width 1) (layer "F.Cu") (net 4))
 (segment (start 124.333 70.231) (end 123.571 70.231) (width 1) (layer "F.Cu") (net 4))
 (segment (start 118.491 105.918) (end 117.602 105.029) (width 1) (layer "F.Cu") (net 4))
 (segment (start 126.492 72.39) (end 126.754 72.128) (width 1) (layer "F.Cu") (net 4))
 (segment (start 120.65 105.918) (end 118.491 105.918) (width 1) (layer "F.Cu") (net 4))
 (segment (start 127.381 75.946) (end 126.492 75.057) (width 1) (layer "F.Cu") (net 4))
 (segment (start 135.636 75.946) (end 127.381 75.946) (width 1) (layer "F.Cu") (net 4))
 (segment (start 127.5 102.3) (end 126.25 101.05) (width 1) (layer "B.Cu") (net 4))
 (segment (start 123.282 105.918) (end 120.65 105.918) (width 1) (layer "B.Cu") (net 4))
 (segment (start 126.25 99) (end 126.25 101.05) (width 1) (layer "B.Cu") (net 4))
 (segment (start 127.5 104.75) (end 127.5 102.3) (width 1) (layer "B.Cu") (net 4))
 (segment (start 127.5 104.75) (end 124.45 104.75) (width 1) (layer "B.Cu") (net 4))
 (segment (start 124.45 104.75) (end 123.282 105.918) (width 1) (layer "B.Cu") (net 4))
 (segment (start 123.622 95.758) (end 125.88 93.5) (width 1) (layer "B.Cu") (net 10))
 (segment (start 120.65 95.758) (end 123.622 95.758) (width 1) (layer "B.Cu") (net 10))
 (segment (start 123.56 90.96) (end 123.278 90.678) (width 1) (layer "B.Cu") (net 9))
 (segment (start 126.492 87.371) (end 126.492 90.348) (width 1) (layer "B.Cu") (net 9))
 (segment (start 126.492 90.348) (end 125.88 90.96) (width 1) (layer "B.Cu") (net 9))
 (segment (start 120.65 90.678) (end 123.278 90.678) (width 1) (layer "B.Cu") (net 9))
 (segment (start 125.88 90.96) (end 123.56 90.96) (width 1) (layer "B.Cu") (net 9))
 (segment (start 120.65 85.598) (end 123.648 82.6) (width 1) (layer "F.Cu") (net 13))
 (segment (start 139 82.6) (end 140 81.6) (width 1) (layer "F.Cu") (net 13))
 (segment (start 123.648 82.6) (end 139 82.6) (width 1) (layer "F.Cu") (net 13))
 (segment (start 140 81.6) (end 140 79.25) (width 1) (layer "F.Cu") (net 13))
 (segment (start 122.555 75.057) (end 122.555 73.914) (width 1) (layer "B.Cu") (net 11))
 (segment (start 122.555 73.914) (end 122.105 73.464) (width 1) (layer "B.Cu") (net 11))
 (segment (start 122.105 73.464) (end 122.105 72.009) (width 1) (layer "B.Cu") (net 11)))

